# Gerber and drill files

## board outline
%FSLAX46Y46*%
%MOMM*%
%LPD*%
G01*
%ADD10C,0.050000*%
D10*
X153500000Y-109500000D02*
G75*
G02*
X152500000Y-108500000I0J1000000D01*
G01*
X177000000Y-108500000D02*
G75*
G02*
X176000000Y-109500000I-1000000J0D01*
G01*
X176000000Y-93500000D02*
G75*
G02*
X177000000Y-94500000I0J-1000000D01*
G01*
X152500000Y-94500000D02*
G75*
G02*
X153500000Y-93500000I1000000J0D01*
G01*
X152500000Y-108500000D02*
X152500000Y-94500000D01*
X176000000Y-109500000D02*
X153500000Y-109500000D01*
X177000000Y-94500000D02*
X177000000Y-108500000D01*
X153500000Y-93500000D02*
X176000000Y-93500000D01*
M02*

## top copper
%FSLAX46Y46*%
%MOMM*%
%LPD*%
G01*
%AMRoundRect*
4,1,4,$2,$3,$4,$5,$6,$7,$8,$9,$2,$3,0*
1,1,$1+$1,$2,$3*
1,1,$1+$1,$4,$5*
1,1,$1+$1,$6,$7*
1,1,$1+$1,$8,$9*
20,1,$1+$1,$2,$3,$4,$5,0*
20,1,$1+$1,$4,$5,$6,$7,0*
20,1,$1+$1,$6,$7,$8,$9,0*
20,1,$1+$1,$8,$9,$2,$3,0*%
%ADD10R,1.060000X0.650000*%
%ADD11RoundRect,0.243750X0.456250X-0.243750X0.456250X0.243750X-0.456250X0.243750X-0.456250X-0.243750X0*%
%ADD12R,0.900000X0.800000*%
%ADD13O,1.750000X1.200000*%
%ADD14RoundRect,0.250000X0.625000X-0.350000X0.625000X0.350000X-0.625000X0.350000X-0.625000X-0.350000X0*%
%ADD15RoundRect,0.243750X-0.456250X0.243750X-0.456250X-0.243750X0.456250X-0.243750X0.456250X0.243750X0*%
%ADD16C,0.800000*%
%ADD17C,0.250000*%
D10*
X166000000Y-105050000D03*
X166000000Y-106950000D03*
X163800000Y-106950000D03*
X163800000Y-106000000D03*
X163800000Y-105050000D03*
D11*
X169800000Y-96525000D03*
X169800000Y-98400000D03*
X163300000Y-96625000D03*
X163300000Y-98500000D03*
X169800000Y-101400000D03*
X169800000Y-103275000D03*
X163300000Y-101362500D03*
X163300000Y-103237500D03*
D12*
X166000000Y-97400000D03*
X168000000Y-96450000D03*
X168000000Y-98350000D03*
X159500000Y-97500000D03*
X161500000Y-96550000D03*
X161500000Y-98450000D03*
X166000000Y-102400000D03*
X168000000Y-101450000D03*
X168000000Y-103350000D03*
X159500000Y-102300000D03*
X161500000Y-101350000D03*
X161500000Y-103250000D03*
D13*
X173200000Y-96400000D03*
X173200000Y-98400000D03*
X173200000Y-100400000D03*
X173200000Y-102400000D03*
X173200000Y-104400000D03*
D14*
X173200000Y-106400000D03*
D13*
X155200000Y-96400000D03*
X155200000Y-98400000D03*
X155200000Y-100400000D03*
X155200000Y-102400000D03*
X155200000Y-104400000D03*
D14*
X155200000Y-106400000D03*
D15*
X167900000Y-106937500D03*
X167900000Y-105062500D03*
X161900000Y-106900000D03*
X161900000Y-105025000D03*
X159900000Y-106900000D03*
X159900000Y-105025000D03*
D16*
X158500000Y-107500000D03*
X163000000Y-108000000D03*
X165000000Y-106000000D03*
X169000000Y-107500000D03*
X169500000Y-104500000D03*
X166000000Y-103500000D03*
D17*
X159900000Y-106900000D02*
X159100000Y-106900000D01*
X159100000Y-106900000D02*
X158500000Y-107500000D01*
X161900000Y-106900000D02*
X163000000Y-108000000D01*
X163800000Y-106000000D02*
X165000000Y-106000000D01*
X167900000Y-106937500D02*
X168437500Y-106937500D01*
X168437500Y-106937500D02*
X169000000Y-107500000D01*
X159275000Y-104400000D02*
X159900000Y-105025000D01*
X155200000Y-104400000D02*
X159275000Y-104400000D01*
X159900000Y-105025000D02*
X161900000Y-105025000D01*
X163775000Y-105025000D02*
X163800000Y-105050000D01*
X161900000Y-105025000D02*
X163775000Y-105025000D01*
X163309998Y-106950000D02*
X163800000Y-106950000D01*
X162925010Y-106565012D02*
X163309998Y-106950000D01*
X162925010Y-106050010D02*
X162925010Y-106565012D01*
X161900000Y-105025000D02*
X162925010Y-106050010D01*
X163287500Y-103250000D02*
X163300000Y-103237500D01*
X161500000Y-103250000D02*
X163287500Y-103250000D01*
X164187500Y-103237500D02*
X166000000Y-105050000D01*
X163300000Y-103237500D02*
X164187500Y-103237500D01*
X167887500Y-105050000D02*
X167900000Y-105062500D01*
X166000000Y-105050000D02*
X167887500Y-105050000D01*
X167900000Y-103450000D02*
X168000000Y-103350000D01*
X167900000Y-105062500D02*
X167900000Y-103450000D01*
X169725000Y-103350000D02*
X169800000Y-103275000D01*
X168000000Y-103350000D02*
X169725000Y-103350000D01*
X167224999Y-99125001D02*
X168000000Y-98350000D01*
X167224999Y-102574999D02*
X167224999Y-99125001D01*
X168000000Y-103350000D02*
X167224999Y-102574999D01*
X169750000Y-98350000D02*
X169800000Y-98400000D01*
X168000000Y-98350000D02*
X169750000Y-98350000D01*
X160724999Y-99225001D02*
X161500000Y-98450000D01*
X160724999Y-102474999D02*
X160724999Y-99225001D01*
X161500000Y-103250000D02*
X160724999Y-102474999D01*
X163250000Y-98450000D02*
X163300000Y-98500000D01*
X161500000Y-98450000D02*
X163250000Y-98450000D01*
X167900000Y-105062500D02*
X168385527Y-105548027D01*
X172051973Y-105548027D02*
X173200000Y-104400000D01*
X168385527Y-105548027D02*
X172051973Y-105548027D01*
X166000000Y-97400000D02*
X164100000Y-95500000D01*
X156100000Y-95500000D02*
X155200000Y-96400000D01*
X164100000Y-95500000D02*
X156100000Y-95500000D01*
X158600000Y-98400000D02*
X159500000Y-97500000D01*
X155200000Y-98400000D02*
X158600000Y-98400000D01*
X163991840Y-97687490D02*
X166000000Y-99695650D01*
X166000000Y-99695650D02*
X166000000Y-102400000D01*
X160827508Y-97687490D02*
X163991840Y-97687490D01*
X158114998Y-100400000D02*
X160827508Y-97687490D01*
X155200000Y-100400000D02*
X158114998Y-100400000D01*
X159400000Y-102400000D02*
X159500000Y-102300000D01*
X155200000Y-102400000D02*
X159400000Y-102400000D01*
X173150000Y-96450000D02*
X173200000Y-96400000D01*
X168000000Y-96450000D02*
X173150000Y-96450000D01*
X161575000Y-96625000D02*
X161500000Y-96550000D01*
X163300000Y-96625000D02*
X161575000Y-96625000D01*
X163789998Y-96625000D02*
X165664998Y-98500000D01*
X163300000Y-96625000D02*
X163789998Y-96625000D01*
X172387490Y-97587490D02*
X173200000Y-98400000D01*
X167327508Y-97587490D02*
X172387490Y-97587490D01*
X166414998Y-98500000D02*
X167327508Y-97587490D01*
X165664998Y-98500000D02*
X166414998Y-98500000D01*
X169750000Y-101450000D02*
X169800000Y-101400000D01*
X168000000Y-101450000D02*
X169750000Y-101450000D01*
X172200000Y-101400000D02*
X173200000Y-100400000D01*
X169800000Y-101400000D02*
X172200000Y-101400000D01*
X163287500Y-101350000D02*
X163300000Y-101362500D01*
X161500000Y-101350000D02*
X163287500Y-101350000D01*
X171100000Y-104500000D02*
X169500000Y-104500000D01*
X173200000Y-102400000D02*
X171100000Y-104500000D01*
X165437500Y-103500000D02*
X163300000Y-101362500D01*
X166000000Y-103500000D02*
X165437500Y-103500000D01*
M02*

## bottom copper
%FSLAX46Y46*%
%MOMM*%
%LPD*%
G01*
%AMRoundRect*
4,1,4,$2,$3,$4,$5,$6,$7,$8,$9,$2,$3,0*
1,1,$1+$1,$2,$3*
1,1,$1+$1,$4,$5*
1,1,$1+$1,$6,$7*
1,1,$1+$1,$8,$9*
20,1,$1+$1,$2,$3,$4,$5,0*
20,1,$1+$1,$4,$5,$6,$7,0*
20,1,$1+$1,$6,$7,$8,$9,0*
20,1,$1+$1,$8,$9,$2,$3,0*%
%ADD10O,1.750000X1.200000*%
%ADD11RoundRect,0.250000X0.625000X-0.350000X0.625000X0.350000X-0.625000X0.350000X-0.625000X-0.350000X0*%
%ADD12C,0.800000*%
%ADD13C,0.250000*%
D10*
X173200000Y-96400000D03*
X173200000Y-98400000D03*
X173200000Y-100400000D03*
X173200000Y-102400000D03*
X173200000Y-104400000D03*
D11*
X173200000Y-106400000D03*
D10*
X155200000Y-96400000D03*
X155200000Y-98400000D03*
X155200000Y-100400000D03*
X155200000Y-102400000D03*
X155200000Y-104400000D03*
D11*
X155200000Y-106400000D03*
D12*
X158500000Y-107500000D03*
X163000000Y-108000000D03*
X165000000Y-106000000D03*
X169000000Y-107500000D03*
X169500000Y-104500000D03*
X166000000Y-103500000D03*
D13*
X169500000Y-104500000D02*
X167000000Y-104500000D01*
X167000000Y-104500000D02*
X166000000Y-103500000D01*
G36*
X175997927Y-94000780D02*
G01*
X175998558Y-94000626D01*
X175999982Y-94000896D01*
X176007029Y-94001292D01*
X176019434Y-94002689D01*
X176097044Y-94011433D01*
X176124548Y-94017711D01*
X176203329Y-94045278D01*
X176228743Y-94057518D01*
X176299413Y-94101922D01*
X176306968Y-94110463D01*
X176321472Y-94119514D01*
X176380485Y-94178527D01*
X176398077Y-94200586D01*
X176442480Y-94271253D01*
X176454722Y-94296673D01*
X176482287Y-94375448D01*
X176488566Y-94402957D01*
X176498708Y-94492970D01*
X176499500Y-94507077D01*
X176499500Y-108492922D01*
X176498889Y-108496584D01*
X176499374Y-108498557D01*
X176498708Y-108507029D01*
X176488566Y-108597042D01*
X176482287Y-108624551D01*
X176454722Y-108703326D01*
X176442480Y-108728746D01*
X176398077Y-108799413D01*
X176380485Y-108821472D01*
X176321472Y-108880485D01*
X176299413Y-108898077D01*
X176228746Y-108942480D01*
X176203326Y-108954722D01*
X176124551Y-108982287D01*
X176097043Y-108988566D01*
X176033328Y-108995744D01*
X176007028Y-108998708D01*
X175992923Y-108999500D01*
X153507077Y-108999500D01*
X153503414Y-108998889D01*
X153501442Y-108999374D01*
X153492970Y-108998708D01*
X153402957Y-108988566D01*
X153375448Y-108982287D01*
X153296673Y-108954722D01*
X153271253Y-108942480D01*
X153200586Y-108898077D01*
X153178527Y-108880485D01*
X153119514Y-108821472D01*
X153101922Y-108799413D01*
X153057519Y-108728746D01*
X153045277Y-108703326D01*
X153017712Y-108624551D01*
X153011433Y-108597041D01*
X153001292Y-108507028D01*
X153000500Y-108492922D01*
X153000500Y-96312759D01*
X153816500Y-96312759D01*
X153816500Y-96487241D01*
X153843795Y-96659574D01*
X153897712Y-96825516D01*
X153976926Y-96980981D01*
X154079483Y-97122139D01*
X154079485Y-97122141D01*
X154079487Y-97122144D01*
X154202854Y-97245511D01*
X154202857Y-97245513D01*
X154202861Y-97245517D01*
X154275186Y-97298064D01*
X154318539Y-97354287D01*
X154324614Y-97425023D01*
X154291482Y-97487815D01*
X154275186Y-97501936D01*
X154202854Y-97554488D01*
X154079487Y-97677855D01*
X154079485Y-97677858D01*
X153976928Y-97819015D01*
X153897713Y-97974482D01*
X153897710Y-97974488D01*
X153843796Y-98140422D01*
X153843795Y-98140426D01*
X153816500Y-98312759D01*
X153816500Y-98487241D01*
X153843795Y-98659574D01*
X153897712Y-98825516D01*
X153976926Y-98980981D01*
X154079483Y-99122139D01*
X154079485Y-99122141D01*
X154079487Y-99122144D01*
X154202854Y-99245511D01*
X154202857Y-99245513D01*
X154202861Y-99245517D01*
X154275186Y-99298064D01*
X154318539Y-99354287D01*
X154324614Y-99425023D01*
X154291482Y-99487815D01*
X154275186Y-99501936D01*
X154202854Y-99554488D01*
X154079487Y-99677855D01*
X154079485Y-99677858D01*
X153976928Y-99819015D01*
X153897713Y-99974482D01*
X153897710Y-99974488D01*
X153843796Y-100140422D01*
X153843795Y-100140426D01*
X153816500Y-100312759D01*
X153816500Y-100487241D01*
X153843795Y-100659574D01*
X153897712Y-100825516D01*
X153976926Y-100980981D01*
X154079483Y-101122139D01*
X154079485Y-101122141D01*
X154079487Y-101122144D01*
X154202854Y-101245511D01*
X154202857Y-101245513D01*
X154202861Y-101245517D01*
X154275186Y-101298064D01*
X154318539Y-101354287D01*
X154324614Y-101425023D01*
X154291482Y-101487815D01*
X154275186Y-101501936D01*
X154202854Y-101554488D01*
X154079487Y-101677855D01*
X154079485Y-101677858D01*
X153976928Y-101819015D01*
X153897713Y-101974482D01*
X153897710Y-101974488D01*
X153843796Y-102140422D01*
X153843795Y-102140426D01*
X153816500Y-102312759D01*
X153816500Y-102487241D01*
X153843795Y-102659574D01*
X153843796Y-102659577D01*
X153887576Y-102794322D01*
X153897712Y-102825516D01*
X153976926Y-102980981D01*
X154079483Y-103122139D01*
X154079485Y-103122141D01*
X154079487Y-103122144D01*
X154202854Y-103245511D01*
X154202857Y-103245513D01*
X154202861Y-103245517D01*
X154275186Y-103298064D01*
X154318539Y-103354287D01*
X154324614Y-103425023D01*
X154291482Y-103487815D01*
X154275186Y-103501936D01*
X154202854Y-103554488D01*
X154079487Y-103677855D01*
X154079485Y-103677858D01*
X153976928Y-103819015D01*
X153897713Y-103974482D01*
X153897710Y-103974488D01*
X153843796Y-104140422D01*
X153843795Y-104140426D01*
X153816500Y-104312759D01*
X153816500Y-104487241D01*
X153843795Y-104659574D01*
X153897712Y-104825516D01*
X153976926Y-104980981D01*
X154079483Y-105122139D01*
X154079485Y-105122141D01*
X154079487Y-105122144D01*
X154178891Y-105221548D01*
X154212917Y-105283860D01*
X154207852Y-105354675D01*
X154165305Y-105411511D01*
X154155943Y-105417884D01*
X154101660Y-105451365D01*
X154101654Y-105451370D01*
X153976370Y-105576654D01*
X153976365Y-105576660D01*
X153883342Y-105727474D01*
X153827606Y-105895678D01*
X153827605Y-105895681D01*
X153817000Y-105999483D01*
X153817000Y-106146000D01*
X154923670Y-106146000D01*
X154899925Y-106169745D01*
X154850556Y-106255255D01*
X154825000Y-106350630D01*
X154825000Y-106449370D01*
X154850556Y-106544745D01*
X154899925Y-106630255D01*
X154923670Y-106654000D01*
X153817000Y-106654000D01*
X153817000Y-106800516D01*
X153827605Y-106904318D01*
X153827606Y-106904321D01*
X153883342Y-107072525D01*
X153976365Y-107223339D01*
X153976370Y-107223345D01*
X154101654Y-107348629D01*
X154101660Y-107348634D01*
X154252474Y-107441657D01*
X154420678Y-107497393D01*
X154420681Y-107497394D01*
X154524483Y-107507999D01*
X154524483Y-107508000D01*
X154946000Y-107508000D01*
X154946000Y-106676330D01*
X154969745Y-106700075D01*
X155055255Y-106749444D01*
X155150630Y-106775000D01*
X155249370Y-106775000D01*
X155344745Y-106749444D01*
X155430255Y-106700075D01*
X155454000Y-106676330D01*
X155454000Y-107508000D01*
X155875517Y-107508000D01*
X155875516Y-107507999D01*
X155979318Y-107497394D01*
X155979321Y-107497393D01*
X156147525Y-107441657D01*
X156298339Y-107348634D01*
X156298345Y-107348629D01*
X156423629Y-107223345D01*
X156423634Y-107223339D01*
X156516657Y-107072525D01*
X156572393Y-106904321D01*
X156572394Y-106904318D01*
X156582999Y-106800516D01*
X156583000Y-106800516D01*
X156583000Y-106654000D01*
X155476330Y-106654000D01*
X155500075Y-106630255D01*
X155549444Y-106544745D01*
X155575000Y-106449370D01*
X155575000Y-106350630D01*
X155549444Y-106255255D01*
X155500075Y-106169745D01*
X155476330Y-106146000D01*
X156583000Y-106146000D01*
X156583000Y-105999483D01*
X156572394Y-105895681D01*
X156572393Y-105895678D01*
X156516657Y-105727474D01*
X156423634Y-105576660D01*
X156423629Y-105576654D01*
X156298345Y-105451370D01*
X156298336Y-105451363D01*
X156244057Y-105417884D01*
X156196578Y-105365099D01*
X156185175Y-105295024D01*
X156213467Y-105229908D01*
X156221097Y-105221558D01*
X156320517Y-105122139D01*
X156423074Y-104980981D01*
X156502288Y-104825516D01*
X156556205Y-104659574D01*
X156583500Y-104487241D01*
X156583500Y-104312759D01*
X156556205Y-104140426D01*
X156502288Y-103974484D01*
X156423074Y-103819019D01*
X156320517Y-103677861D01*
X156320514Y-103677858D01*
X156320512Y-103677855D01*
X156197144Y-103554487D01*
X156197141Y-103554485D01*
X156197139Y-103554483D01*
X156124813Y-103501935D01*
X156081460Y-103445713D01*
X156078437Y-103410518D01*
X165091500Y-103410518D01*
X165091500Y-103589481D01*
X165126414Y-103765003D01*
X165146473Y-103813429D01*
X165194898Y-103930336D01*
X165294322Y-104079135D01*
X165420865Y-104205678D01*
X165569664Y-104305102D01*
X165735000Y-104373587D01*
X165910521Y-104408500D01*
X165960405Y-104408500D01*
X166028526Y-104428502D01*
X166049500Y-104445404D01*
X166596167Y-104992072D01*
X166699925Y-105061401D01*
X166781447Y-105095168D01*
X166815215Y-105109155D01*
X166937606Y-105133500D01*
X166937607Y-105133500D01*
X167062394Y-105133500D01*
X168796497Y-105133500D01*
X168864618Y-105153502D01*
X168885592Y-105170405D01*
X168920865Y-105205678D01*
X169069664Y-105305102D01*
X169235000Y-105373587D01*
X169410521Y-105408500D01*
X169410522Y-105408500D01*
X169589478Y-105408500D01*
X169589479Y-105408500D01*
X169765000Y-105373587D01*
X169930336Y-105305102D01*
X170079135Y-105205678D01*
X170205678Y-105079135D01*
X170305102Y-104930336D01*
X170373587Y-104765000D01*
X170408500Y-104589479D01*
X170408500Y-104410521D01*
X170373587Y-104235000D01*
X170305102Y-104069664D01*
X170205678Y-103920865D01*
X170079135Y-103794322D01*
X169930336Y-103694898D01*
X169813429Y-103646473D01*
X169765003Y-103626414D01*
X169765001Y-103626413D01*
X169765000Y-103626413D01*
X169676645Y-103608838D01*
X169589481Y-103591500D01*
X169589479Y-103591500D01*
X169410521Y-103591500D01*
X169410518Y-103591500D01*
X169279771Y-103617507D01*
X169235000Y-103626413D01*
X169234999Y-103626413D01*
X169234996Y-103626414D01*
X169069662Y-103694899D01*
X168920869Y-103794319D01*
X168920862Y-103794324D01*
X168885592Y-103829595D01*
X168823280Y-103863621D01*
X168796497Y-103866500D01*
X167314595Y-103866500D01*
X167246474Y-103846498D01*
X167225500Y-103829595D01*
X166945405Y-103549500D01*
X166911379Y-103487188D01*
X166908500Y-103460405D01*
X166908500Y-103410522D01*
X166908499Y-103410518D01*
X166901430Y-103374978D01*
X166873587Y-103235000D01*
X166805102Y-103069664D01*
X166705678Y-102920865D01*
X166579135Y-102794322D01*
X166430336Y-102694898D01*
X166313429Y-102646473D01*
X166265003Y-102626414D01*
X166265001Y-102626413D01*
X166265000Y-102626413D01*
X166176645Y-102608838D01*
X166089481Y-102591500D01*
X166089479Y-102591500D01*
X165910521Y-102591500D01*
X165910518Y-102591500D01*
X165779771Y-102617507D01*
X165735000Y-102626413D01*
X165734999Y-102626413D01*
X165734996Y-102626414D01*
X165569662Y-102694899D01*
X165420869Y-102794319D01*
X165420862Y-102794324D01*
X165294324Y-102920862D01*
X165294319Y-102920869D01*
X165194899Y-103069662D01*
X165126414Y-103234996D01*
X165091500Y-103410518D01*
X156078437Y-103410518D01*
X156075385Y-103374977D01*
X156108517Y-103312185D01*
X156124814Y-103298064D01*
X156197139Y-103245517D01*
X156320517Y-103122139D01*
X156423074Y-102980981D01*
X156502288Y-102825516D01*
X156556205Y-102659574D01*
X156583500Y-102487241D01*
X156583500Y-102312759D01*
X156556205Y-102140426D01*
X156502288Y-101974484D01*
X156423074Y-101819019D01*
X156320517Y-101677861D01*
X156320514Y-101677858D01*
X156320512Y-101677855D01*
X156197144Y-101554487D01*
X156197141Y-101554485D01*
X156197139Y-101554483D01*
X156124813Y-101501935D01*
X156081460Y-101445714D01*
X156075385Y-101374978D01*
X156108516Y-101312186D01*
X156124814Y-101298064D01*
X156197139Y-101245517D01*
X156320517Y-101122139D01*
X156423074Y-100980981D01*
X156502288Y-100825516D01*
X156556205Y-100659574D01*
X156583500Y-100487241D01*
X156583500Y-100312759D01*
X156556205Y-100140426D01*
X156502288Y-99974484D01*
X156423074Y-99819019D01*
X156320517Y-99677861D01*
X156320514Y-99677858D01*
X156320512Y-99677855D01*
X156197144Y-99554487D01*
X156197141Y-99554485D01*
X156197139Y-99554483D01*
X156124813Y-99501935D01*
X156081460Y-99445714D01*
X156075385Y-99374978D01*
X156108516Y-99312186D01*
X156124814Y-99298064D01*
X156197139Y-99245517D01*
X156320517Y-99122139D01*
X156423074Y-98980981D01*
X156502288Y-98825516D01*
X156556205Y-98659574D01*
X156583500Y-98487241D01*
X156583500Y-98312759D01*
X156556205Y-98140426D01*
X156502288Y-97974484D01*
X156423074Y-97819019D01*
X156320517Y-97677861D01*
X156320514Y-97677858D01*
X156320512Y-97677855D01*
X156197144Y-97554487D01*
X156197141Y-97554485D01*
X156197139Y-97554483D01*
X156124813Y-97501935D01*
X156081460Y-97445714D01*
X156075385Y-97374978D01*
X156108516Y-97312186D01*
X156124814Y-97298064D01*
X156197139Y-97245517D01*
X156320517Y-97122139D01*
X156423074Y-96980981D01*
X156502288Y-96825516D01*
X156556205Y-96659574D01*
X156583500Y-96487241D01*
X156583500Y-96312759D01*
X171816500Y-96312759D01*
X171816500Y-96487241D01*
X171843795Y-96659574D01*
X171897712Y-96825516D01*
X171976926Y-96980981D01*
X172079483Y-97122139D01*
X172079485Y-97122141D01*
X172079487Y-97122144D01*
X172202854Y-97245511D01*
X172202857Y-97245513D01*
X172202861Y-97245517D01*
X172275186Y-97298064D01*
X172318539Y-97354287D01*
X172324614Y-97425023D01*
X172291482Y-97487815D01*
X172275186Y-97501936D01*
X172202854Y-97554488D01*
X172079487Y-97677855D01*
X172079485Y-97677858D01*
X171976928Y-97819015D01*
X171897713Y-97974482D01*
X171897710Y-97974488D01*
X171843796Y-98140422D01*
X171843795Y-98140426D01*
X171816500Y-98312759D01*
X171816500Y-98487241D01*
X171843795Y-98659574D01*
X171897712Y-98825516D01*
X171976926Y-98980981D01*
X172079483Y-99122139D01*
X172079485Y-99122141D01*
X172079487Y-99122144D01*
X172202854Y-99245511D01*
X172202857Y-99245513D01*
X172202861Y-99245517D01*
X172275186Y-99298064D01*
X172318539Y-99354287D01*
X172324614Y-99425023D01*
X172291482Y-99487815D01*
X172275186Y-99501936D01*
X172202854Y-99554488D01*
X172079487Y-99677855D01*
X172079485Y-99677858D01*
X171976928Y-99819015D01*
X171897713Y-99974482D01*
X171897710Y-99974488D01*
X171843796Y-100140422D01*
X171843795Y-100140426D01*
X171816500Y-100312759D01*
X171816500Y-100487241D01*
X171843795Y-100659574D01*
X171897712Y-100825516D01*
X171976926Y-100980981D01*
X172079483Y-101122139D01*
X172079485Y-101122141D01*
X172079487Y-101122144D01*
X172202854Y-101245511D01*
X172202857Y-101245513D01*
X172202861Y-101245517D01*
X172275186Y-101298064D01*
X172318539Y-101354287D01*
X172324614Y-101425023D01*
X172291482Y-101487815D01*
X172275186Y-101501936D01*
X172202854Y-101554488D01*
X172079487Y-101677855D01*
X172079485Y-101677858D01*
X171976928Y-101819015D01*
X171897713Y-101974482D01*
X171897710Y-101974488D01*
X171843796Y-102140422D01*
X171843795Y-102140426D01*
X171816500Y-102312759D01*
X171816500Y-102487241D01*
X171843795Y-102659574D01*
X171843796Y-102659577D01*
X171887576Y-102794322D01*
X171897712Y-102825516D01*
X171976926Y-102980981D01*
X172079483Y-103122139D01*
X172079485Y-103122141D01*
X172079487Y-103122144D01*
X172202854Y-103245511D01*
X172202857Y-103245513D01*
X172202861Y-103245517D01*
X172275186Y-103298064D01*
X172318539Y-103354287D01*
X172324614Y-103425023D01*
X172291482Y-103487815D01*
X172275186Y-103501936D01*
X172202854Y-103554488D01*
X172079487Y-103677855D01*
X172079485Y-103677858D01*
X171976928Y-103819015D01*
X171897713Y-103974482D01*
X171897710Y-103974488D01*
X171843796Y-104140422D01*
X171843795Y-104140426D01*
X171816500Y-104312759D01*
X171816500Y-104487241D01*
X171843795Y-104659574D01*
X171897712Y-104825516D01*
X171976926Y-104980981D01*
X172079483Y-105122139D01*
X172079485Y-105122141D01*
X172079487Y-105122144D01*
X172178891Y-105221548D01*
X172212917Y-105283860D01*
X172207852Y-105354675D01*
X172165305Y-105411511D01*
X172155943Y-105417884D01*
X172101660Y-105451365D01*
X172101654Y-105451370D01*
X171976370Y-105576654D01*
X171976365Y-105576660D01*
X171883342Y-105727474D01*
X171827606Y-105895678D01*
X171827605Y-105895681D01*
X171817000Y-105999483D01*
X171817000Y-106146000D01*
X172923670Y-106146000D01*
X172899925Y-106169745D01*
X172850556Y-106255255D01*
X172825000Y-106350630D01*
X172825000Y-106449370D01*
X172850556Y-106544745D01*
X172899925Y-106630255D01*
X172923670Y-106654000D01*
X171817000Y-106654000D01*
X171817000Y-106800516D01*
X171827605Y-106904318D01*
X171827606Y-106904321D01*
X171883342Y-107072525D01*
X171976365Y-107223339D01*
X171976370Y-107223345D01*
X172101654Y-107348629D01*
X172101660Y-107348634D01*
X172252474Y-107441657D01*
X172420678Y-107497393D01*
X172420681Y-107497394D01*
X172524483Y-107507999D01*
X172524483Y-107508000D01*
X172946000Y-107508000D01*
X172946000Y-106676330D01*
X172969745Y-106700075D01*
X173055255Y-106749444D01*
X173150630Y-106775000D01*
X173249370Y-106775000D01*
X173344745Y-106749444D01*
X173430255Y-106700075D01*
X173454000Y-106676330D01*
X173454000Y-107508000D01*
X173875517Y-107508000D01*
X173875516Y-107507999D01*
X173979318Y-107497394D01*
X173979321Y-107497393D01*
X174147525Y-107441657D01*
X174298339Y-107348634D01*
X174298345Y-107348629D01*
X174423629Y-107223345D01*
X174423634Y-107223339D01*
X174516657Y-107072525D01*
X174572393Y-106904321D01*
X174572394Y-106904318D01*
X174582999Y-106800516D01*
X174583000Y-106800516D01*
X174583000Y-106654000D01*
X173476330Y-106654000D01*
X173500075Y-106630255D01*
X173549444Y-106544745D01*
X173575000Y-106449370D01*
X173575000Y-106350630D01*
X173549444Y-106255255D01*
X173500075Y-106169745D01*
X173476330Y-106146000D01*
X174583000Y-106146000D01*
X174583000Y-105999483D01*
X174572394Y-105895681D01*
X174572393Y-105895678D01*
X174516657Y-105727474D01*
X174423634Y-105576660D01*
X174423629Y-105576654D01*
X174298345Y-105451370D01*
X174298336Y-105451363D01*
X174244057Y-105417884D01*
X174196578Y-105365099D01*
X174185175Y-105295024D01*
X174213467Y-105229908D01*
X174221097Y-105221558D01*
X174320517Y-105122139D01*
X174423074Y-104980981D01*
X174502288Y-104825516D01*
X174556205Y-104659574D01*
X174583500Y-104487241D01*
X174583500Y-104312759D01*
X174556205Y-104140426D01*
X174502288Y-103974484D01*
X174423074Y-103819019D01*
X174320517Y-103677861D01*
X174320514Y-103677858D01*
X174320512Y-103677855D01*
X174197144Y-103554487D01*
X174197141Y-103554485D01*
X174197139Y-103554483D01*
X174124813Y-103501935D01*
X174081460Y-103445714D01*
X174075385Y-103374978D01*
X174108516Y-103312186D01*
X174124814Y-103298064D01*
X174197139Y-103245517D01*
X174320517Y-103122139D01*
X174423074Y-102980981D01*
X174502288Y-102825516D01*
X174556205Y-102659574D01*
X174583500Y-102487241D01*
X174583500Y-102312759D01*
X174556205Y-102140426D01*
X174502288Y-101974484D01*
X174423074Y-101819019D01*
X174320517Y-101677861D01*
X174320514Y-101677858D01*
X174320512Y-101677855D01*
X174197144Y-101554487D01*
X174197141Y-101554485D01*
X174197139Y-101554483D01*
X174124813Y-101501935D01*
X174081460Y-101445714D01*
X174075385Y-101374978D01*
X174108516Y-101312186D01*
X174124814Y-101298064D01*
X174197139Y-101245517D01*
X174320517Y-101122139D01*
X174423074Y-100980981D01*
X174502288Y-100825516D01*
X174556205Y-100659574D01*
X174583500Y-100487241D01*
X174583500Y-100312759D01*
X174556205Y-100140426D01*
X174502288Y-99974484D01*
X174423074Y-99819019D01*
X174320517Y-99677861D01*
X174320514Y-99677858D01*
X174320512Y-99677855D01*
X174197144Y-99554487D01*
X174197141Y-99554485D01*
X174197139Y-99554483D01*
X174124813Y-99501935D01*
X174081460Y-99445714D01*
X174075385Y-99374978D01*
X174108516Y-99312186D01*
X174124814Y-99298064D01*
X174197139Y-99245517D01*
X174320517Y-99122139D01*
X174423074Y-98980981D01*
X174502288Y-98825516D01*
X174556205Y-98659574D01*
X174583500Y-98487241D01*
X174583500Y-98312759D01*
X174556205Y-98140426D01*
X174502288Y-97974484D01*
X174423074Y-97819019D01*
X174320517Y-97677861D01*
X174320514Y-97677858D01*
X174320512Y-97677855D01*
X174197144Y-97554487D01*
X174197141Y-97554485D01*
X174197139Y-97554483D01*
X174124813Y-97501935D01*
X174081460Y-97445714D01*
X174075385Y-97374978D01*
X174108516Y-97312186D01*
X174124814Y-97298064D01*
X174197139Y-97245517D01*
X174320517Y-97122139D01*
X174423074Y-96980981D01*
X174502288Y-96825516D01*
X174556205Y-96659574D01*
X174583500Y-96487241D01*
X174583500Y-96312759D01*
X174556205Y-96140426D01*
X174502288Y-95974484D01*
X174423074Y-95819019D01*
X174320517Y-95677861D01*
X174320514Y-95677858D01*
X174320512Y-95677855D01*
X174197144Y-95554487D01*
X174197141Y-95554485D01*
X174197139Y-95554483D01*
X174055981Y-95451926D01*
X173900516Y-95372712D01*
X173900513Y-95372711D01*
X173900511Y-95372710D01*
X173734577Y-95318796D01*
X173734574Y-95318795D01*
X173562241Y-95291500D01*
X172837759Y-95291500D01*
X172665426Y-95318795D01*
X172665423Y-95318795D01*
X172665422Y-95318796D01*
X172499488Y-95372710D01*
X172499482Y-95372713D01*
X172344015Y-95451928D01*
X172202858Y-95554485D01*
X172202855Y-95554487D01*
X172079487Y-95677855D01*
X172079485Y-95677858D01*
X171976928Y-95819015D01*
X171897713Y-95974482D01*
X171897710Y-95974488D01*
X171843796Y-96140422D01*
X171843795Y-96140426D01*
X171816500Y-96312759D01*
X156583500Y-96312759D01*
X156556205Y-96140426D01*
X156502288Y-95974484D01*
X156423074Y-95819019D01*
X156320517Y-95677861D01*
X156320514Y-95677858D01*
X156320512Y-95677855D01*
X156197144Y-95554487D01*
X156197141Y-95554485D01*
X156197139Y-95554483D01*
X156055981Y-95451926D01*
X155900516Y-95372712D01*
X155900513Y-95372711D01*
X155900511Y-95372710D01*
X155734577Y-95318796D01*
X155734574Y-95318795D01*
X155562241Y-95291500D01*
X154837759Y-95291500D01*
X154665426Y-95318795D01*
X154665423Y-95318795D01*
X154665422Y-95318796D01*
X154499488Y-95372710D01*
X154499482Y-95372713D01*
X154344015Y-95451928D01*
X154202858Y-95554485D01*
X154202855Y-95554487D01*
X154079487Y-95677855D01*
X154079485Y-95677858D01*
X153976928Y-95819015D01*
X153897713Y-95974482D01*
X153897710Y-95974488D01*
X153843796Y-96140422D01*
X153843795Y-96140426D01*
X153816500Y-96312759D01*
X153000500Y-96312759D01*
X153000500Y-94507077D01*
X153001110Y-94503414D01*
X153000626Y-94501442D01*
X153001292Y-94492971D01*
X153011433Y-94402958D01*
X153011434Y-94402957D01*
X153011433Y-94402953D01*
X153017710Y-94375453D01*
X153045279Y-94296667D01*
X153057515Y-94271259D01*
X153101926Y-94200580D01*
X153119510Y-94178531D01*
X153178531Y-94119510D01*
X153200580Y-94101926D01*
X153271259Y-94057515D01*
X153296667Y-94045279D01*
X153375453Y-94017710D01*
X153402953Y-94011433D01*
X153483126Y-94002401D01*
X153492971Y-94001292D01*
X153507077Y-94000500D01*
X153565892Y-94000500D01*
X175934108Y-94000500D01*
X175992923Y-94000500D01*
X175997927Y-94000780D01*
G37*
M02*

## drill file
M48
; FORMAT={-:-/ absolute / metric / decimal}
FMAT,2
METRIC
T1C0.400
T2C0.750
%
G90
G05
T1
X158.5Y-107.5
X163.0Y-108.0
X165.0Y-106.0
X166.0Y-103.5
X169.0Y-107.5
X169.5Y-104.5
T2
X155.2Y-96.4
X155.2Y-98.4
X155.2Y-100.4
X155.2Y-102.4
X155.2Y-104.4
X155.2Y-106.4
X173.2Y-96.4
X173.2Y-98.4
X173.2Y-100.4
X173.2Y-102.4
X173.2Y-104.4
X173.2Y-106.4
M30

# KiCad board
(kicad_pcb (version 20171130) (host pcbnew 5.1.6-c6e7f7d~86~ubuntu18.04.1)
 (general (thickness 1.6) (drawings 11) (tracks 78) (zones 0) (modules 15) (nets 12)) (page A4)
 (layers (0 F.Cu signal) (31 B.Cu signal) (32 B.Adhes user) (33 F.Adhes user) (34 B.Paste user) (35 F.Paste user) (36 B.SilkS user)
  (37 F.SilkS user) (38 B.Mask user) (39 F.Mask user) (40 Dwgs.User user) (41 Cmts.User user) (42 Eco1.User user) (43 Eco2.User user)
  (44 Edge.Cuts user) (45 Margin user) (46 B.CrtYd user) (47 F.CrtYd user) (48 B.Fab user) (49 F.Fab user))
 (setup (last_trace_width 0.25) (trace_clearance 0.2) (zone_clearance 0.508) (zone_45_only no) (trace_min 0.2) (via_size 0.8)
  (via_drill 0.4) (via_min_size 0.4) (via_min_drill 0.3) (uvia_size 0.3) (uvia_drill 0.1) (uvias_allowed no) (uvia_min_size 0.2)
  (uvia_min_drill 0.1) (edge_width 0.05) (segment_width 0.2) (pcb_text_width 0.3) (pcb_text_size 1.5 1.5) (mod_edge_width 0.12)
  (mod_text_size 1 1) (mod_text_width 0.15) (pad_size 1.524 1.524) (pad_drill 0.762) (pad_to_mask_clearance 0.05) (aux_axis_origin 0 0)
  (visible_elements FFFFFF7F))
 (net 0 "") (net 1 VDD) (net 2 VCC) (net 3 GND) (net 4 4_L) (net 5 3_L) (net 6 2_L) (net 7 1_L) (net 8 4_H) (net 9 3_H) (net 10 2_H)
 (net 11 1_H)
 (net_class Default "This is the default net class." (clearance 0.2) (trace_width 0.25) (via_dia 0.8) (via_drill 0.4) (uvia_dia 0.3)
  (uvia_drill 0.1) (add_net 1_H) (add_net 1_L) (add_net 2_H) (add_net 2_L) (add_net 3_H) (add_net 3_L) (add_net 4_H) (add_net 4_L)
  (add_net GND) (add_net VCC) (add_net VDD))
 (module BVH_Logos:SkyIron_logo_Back (layer F.Cu) (at 164 99)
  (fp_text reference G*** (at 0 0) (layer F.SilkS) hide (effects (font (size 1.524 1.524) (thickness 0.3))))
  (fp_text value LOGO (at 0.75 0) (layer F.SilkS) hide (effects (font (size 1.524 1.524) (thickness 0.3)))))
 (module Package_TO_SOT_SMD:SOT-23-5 (layer F.Cu) (at 164.9 106)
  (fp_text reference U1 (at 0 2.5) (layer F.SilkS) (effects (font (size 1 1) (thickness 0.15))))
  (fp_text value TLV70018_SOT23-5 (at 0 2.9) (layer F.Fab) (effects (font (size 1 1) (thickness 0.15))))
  (pad 5 smd rect (at 1.1 -0.95) (size 1.06 0.65) (layers F.Cu F.Paste F.Mask) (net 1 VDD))
  (pad 4 smd rect (at 1.1 0.95) (size 1.06 0.65) (layers F.Cu F.Paste F.Mask))
  (pad 3 smd rect (at -1.1 0.95) (size 1.06 0.65) (layers F.Cu F.Paste F.Mask) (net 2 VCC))
  (pad 2 smd rect (at -1.1 0) (size 1.06 0.65) (layers F.Cu F.Paste F.Mask) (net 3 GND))
  (pad 1 smd rect (at -1.1 -0.95) (size 1.06 0.65) (layers F.Cu F.Paste F.Mask) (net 2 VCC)))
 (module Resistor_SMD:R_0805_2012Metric (layer F.Cu) (at 169.8 97.4625 90)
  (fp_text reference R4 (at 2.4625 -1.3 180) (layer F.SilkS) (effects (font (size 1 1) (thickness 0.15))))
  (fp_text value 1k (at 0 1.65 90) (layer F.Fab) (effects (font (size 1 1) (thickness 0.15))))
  (pad 2 smd roundrect (at 0.9375 0 90) (size 0.975 1.4) (layers F.Cu F.Paste F.Mask) (roundrect_rratio 0.25) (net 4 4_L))
  (pad 1 smd roundrect (at -0.9375 0 90) (size 0.975 1.4) (layers F.Cu F.Paste F.Mask) (roundrect_rratio 0.25) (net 1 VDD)))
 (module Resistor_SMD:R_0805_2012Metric (layer F.Cu) (at 163.3 97.5625 90)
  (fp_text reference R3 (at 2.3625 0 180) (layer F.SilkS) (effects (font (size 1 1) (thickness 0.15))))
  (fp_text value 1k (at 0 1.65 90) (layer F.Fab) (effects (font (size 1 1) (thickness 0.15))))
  (pad 2 smd roundrect (at 0.9375 0 90) (size 0.975 1.4) (layers F.Cu F.Paste F.Mask) (roundrect_rratio 0.25) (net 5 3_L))
  (pad 1 smd roundrect (at -0.9375 0 90) (size 0.975 1.4) (layers F.Cu F.Paste F.Mask) (roundrect_rratio 0.25) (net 1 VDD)))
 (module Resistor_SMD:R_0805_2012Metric (layer F.Cu) (at 169.8 102.3375 90)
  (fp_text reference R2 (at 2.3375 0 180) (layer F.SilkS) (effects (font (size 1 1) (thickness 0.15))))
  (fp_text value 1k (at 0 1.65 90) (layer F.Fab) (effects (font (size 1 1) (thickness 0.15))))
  (pad 2 smd roundrect (at 0.9375 0 90) (size 0.975 1.4) (layers F.Cu F.Paste F.Mask) (roundrect_rratio 0.25) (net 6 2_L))
  (pad 1 smd roundrect (at -0.9375 0 90) (size 0.975 1.4) (layers F.Cu F.Paste F.Mask) (roundrect_rratio 0.25) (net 1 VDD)))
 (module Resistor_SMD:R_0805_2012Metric (layer F.Cu) (at 163.3 102.3 90)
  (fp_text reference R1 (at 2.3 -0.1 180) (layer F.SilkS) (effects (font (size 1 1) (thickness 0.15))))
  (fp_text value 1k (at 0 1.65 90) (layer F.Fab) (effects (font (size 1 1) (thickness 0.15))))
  (pad 2 smd roundrect (at 0.9375 0 90) (size 0.975 1.4) (layers F.Cu F.Paste F.Mask) (roundrect_rratio 0.25) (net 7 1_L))
  (pad 1 smd roundrect (at -0.9375 0 90) (size 0.975 1.4) (layers F.Cu F.Paste F.Mask) (roundrect_rratio 0.25) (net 1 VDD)))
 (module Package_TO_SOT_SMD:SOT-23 (layer F.Cu) (at 167 97.4 180)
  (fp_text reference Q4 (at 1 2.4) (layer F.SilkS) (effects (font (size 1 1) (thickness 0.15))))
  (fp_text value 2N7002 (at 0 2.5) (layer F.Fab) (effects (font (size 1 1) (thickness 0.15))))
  (pad 3 smd rect (at 1 0 180) (size 0.9 0.8) (layers F.Cu F.Paste F.Mask) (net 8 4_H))
  (pad 2 smd rect (at -1 0.95 180) (size 0.9 0.8) (layers F.Cu F.Paste F.Mask) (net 4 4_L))
  (pad 1 smd rect (at -1 -0.95 180) (size 0.9 0.8) (layers F.Cu F.Paste F.Mask) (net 1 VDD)))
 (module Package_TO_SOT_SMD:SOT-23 (layer F.Cu) (at 160.5 97.5 180)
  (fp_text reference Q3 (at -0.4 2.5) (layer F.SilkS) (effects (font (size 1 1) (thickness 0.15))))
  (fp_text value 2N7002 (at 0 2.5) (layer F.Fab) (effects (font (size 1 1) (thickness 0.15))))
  (pad 3 smd rect (at 1 0 180) (size 0.9 0.8) (layers F.Cu F.Paste F.Mask) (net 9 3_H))
  (pad 2 smd rect (at -1 0.95 180) (size 0.9 0.8) (layers F.Cu F.Paste F.Mask) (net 5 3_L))
  (pad 1 smd rect (at -1 -0.95 180) (size 0.9 0.8) (layers F.Cu F.Paste F.Mask) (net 1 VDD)))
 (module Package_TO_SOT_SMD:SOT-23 (layer F.Cu) (at 167 102.4 180)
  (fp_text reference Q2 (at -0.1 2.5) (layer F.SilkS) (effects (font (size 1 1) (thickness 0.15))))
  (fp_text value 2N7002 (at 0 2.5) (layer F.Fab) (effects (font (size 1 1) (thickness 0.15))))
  (pad 3 smd rect (at 1 0 180) (size 0.9 0.8) (layers F.Cu F.Paste F.Mask) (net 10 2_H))
  (pad 2 smd rect (at -1 0.95 180) (size 0.9 0.8) (layers F.Cu F.Paste F.Mask) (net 6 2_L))
  (pad 1 smd rect (at -1 -0.95 180) (size 0.9 0.8) (layers F.Cu F.Paste F.Mask) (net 1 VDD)))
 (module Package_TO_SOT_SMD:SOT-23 (layer F.Cu) (at 160.5 102.3 180)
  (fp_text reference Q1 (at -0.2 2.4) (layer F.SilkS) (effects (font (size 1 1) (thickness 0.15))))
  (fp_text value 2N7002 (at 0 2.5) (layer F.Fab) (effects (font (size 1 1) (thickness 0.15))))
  (pad 3 smd rect (at 1 0 180) (size 0.9 0.8) (layers F.Cu F.Paste F.Mask) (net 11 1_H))
  (pad 2 smd rect (at -1 0.95 180) (size 0.9 0.8) (layers F.Cu F.Paste F.Mask) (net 7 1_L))
  (pad 1 smd rect (at -1 -0.95 180) (size 0.9 0.8) (layers F.Cu F.Paste F.Mask) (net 1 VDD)))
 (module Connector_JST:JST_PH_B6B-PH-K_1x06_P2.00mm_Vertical (layer F.Cu) (at 173.2 106.4 90)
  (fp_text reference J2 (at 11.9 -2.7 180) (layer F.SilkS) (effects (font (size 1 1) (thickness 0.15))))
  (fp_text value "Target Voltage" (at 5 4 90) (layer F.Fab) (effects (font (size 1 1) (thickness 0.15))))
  (pad 6 thru_hole oval (at 10 0 90) (size 1.2 1.75) (drill 0.75) (layers *.Cu *.Mask) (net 4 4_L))
  (pad 5 thru_hole oval (at 8 0 90) (size 1.2 1.75) (drill 0.75) (layers *.Cu *.Mask) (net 5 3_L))
  (pad 4 thru_hole oval (at 6 0 90) (size 1.2 1.75) (drill 0.75) (layers *.Cu *.Mask) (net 6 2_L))
  (pad 3 thru_hole oval (at 4 0 90) (size 1.2 1.75) (drill 0.75) (layers *.Cu *.Mask) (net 7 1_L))
  (pad 2 thru_hole oval (at 2 0 90) (size 1.2 1.75) (drill 0.75) (layers *.Cu *.Mask) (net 1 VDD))
  (pad 1 thru_hole roundrect (at 0 0 90) (size 1.2 1.75) (drill 0.75) (layers *.Cu *.Mask) (roundrect_rratio 0.208333) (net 3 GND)))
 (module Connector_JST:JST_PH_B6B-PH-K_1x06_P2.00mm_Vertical (layer F.Cu) (at 155.2 106.4 90)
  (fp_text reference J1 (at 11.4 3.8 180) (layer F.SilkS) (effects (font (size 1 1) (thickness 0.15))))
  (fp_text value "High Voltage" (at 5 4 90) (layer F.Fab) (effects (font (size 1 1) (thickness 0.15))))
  (pad 6 thru_hole oval (at 10 0 90) (size 1.2 1.75) (drill 0.75) (layers *.Cu *.Mask) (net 8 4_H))
  (pad 5 thru_hole oval (at 8 0 90) (size 1.2 1.75) (drill 0.75) (layers *.Cu *.Mask) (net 9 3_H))
  (pad 4 thru_hole oval (at 6 0 90) (size 1.2 1.75) (drill 0.75) (layers *.Cu *.Mask) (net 10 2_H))
  (pad 3 thru_hole oval (at 4 0 90) (size 1.2 1.75) (drill 0.75) (layers *.Cu *.Mask) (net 11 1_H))
  (pad 2 thru_hole oval (at 2 0 90) (size 1.2 1.75) (drill 0.75) (layers *.Cu *.Mask) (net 2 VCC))
  (pad 1 thru_hole roundrect (at 0 0 90) (size 1.2 1.75) (drill 0.75) (layers *.Cu *.Mask) (roundrect_rratio 0.208333) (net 3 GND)))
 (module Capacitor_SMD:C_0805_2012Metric (layer F.Cu) (at 167.9 106 270)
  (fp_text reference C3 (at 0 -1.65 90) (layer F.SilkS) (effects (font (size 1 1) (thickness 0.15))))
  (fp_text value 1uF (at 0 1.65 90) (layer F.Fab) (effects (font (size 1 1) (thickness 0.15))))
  (pad 2 smd roundrect (at 0.9375 0 270) (size 0.975 1.4) (layers F.Cu F.Paste F.Mask) (roundrect_rratio 0.25) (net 3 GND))
  (pad 1 smd roundrect (at -0.9375 0 270) (size 0.975 1.4) (layers F.Cu F.Paste F.Mask) (roundrect_rratio 0.25) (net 1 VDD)))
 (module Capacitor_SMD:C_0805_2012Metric (layer F.Cu) (at 161.9 105.9625 270)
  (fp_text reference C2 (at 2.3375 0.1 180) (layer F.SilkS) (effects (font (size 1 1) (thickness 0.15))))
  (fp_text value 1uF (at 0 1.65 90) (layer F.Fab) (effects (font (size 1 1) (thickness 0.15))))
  (pad 2 smd roundrect (at 0.9375 0 270) (size 0.975 1.4) (layers F.Cu F.Paste F.Mask) (roundrect_rratio 0.25) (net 3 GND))
  (pad 1 smd roundrect (at -0.9375 0 270) (size 0.975 1.4) (layers F.Cu F.Paste F.Mask) (roundrect_rratio 0.25) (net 2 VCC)))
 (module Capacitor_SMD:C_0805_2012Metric (layer F.Cu) (at 159.9 105.9625 270)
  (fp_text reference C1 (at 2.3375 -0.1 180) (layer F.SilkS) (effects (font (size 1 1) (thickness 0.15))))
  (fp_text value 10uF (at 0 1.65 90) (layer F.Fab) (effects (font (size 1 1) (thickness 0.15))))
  (pad 2 smd roundrect (at 0.9375 0 270) (size 0.975 1.4) (layers F.Cu F.Paste F.Mask) (roundrect_rratio 0.25) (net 3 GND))
  (pad 1 smd roundrect (at -0.9375 0 270) (size 0.975 1.4) (layers F.Cu F.Paste F.Mask) (roundrect_rratio 0.25) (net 2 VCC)))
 (gr_arc (start 153.5 108.5) (end 152.5 108.5) (angle -90) (layer Edge.Cuts) (width 0.05))
 (gr_arc (start 176 108.5) (end 176 109.5) (angle -90) (layer Edge.Cuts) (width 0.05))
 (gr_arc (start 176 94.5) (end 177 94.5) (angle -90) (layer Edge.Cuts) (width 0.05))
 (gr_arc (start 153.5 94.5) (end 153.5 93.5) (angle -90) (layer Edge.Cuts) (width 0.05))
 (gr_line (start 152.5 108.5) (end 152.5 94.5) (layer Edge.Cuts) (width 0.05))
 (gr_line (start 176 109.5) (end 153.5 109.5) (layer Edge.Cuts) (width 0.05))
 (gr_line (start 177 94.5) (end 177 108.5) (layer Edge.Cuts) (width 0.05))
 (gr_line (start 153.5 93.5) (end 176 93.5) (layer Edge.Cuts) (width 0.05))
 (via (at 158.5 107.5) (size 0.8) (drill 0.4) (layers F.Cu B.Cu) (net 3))
 (segment (start 159.9 106.9) (end 159.1 106.9) (width 0.25) (layer F.Cu) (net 3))
 (segment (start 159.1 106.9) (end 158.5 107.5) (width 0.25) (layer F.Cu) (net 3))
 (via (at 163 108) (size 0.8) (drill 0.4) (layers F.Cu B.Cu) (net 3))
 (segment (start 161.9 106.9) (end 163 108) (width 0.25) (layer F.Cu) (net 3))
 (via (at 165 106) (size 0.8) (drill 0.4) (layers F.Cu B.Cu) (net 3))
 (segment (start 163.8 106) (end 165 106) (width 0.25) (layer F.Cu) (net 3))
 (via (at 169 107.5) (size 0.8) (drill 0.4) (layers F.Cu B.Cu) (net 3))
 (segment (start 167.9 106.9375) (end 168.4375 106.9375) (width 0.25) (layer F.Cu) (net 3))
 (segment (start 168.4375 106.9375) (end 169 107.5) (width 0.25) (layer F.Cu) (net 3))
 (segment (start 159.275 104.4) (end 159.9 105.025) (width 0.25) (layer F.Cu) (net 2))
 (segment (start 155.2 104.4) (end 159.275 104.4) (width 0.25) (layer F.Cu) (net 2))
 (segment (start 159.9 105.025) (end 161.9 105.025) (width 0.25) (layer F.Cu) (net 2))
 (segment (start 163.775 105.025) (end 163.8 105.05) (width 0.25) (layer F.Cu) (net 2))
 (segment (start 161.9 105.025) (end 163.775 105.025) (width 0.25) (layer F.Cu) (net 2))
 (segment (start 163.309998 106.95) (end 163.8 106.95) (width 0.25) (layer F.Cu) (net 2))
 (segment (start 162.92501 106.565012) (end 163.309998 106.95) (width 0.25) (layer F.Cu) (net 2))
 (segment (start 162.92501 106.05001) (end 162.92501 106.565012) (width 0.25) (layer F.Cu) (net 2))
 (segment (start 161.9 105.025) (end 162.92501 106.05001) (width 0.25) (layer F.Cu) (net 2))
 (segment (start 163.2875 103.25) (end 163.3 103.2375) (width 0.25) (layer F.Cu) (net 1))
 (segment (start 161.5 103.25) (end 163.2875 103.25) (width 0.25) (layer F.Cu) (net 1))
 (segment (start 164.1875 103.2375) (end 166 105.05) (width 0.25) (layer F.Cu) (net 1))
 (segment (start 163.3 103.2375) (end 164.1875 103.2375) (width 0.25) (layer F.Cu) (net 1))
 (segment (start 167.8875 105.05) (end 167.9 105.0625) (width 0.25) (layer F.Cu) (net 1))
 (segment (start 166 105.05) (end 167.8875 105.05) (width 0.25) (layer F.Cu) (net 1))
 (segment (start 167.9 103.45) (end 168 103.35) (width 0.25) (layer F.Cu) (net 1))
 (segment (start 167.9 105.0625) (end 167.9 103.45) (width 0.25) (layer F.Cu) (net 1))
 (segment (start 169.725 103.35) (end 169.8 103.275) (width 0.25) (layer F.Cu) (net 1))
 (segment (start 168 103.35) (end 169.725 103.35) (width 0.25) (layer F.Cu) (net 1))
 (segment (start 167.224999 99.125001) (end 168 98.35) (width 0.25) (layer F.Cu) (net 1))
 (segment (start 167.224999 102.574999) (end 167.224999 99.125001) (width 0.25) (layer F.Cu) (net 1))
 (segment (start 168 103.35) (end 167.224999 102.574999) (width 0.25) (layer F.Cu) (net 1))
 (segment (start 169.75 98.35) (end 169.8 98.4) (width 0.25) (layer F.Cu) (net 1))
 (segment (start 168 98.35) (end 169.75 98.35) (width 0.25) (layer F.Cu) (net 1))
 (segment (start 160.724999 99.225001) (end 161.5 98.45) (width 0.25) (layer F.Cu) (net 1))
 (segment (start 160.724999 102.474999) (end 160.724999 99.225001) (width 0.25) (layer F.Cu) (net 1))
 (segment (start 161.5 103.25) (end 160.724999 102.474999) (width 0.25) (layer F.Cu) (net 1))
 (segment (start 163.25 98.45) (end 163.3 98.5) (width 0.25) (layer F.Cu) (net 1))
 (segment (start 161.5 98.45) (end 163.25 98.45) (width 0.25) (layer F.Cu) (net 1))
 (segment (start 167.9 105.0625) (end 168.385527 105.548027) (width 0.25) (layer F.Cu) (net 1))
 (segment (start 172.051973 105.548027) (end 173.2 104.4) (width 0.25) (layer F.Cu) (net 1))
 (segment (start 168.385527 105.548027) (end 172.051973 105.548027) (width 0.25) (layer F.Cu) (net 1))
 (segment (start 166 97.4) (end 164.1 95.5) (width 0.25) (layer F.Cu) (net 8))
 (segment (start 156.1 95.5) (end 155.2 96.4) (width 0.25) (layer F.Cu) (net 8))
 (segment (start 164.1 95.5) (end 156.1 95.5) (width 0.25) (layer F.Cu) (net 8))
 (segment (start 158.6 98.4) (end 159.5 97.5) (width 0.25) (layer F.Cu) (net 9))
 (segment (start 155.2 98.4) (end 158.6 98.4) (width 0.25) (layer F.Cu) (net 9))
 (segment (start 163.99184 97.68749) (end 166 99.69565) (width 0.25) (layer F.Cu) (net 10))
 (segment (start 166 99.69565) (end 166 102.4) (width 0.25) (layer F.Cu) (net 10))
 (segment (start 160.827508 97.68749) (end 163.99184 97.68749) (width 0.25) (layer F.Cu) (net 10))
 (segment (start 158.114998 100.4) (end 160.827508 97.68749) (width 0.25) (layer F.Cu) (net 10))
 (segment (start 155.2 100.4) (end 158.114998 100.4) (width 0.25) (layer F.Cu) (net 10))
 (segment (start 159.4 102.4) (end 159.5 102.3) (width 0.25) (layer F.Cu) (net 11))
 (segment (start 155.2 102.4) (end 159.4 102.4) (width 0.25) (layer F.Cu) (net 11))
 (segment (start 173.15 96.45) (end 173.2 96.4) (width 0.25) (layer F.Cu) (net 4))
 (segment (start 168 96.45) (end 173.15 96.45) (width 0.25) (layer F.Cu) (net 4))
 (segment (start 161.575 96.625) (end 161.5 96.55) (width 0.25) (layer F.Cu) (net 5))
 (segment (start 163.3 96.625) (end 161.575 96.625) (width 0.25) (layer F.Cu) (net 5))
 (segment (start 163.789998 96.625) (end 165.664998 98.5) (width 0.25) (layer F.Cu) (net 5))
 (segment (start 163.3 96.625) (end 163.789998 96.625) (width 0.25) (layer F.Cu) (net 5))
 (segment (start 172.38749 97.58749) (end 173.2 98.4) (width 0.25) (layer F.Cu) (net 5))
 (segment (start 167.327508 97.58749) (end 172.38749 97.58749) (width 0.25) (layer F.Cu) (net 5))
 (segment (start 166.414998 98.5) (end 167.327508 97.58749) (width 0.25) (layer F.Cu) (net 5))
 (segment (start 165.664998 98.5) (end 166.414998 98.5) (width 0.25) (layer F.Cu) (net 5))
 (segment (start 169.75 101.45) (end 169.8 101.4) (width 0.25) (layer F.Cu) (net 6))
 (segment (start 168 101.45) (end 169.75 101.45) (width 0.25) (layer F.Cu) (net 6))
 (segment (start 172.2 101.4) (end 173.2 100.4) (width 0.25) (layer F.Cu) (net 6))
 (segment (start 169.8 101.4) (end 172.2 101.4) (width 0.25) (layer F.Cu) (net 6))
 (segment (start 163.2875 101.35) (end 163.3 101.3625) (width 0.25) (layer F.Cu) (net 7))
 (segment (start 161.5 101.35) (end 163.2875 101.35) (width 0.25) (layer F.Cu) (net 7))
 (segment (start 171.1 104.5) (end 169.5 104.5) (width 0.25) (layer F.Cu) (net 7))
 (segment (start 173.2 102.4) (end 171.1 104.5) (width 0.25) (layer F.Cu) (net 7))
 (via (at 169.5 104.5) (size 0.8) (drill 0.4) (layers F.Cu B.Cu) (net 7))
 (via (at 166 103.5) (size 0.8) (drill 0.4) (layers F.Cu B.Cu) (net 7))
 (segment (start 169.5 104.5) (end 167 104.5) (width 0.25) (layer B.Cu) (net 7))
 (segment (start 167 104.5) (end 166 103.5) (width 0.25) (layer B.Cu) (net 7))
 (segment (start 165.4375 103.5) (end 163.3 101.3625) (width 0.25) (layer F.Cu) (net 7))
 (segment (start 166 103.5) (end 165.4375 103.5) (width 0.25) (layer F.Cu) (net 7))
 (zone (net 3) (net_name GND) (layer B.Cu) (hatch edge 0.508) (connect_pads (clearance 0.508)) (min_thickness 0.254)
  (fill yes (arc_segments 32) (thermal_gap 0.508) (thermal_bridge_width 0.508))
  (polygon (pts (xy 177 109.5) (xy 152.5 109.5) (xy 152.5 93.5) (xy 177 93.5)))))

